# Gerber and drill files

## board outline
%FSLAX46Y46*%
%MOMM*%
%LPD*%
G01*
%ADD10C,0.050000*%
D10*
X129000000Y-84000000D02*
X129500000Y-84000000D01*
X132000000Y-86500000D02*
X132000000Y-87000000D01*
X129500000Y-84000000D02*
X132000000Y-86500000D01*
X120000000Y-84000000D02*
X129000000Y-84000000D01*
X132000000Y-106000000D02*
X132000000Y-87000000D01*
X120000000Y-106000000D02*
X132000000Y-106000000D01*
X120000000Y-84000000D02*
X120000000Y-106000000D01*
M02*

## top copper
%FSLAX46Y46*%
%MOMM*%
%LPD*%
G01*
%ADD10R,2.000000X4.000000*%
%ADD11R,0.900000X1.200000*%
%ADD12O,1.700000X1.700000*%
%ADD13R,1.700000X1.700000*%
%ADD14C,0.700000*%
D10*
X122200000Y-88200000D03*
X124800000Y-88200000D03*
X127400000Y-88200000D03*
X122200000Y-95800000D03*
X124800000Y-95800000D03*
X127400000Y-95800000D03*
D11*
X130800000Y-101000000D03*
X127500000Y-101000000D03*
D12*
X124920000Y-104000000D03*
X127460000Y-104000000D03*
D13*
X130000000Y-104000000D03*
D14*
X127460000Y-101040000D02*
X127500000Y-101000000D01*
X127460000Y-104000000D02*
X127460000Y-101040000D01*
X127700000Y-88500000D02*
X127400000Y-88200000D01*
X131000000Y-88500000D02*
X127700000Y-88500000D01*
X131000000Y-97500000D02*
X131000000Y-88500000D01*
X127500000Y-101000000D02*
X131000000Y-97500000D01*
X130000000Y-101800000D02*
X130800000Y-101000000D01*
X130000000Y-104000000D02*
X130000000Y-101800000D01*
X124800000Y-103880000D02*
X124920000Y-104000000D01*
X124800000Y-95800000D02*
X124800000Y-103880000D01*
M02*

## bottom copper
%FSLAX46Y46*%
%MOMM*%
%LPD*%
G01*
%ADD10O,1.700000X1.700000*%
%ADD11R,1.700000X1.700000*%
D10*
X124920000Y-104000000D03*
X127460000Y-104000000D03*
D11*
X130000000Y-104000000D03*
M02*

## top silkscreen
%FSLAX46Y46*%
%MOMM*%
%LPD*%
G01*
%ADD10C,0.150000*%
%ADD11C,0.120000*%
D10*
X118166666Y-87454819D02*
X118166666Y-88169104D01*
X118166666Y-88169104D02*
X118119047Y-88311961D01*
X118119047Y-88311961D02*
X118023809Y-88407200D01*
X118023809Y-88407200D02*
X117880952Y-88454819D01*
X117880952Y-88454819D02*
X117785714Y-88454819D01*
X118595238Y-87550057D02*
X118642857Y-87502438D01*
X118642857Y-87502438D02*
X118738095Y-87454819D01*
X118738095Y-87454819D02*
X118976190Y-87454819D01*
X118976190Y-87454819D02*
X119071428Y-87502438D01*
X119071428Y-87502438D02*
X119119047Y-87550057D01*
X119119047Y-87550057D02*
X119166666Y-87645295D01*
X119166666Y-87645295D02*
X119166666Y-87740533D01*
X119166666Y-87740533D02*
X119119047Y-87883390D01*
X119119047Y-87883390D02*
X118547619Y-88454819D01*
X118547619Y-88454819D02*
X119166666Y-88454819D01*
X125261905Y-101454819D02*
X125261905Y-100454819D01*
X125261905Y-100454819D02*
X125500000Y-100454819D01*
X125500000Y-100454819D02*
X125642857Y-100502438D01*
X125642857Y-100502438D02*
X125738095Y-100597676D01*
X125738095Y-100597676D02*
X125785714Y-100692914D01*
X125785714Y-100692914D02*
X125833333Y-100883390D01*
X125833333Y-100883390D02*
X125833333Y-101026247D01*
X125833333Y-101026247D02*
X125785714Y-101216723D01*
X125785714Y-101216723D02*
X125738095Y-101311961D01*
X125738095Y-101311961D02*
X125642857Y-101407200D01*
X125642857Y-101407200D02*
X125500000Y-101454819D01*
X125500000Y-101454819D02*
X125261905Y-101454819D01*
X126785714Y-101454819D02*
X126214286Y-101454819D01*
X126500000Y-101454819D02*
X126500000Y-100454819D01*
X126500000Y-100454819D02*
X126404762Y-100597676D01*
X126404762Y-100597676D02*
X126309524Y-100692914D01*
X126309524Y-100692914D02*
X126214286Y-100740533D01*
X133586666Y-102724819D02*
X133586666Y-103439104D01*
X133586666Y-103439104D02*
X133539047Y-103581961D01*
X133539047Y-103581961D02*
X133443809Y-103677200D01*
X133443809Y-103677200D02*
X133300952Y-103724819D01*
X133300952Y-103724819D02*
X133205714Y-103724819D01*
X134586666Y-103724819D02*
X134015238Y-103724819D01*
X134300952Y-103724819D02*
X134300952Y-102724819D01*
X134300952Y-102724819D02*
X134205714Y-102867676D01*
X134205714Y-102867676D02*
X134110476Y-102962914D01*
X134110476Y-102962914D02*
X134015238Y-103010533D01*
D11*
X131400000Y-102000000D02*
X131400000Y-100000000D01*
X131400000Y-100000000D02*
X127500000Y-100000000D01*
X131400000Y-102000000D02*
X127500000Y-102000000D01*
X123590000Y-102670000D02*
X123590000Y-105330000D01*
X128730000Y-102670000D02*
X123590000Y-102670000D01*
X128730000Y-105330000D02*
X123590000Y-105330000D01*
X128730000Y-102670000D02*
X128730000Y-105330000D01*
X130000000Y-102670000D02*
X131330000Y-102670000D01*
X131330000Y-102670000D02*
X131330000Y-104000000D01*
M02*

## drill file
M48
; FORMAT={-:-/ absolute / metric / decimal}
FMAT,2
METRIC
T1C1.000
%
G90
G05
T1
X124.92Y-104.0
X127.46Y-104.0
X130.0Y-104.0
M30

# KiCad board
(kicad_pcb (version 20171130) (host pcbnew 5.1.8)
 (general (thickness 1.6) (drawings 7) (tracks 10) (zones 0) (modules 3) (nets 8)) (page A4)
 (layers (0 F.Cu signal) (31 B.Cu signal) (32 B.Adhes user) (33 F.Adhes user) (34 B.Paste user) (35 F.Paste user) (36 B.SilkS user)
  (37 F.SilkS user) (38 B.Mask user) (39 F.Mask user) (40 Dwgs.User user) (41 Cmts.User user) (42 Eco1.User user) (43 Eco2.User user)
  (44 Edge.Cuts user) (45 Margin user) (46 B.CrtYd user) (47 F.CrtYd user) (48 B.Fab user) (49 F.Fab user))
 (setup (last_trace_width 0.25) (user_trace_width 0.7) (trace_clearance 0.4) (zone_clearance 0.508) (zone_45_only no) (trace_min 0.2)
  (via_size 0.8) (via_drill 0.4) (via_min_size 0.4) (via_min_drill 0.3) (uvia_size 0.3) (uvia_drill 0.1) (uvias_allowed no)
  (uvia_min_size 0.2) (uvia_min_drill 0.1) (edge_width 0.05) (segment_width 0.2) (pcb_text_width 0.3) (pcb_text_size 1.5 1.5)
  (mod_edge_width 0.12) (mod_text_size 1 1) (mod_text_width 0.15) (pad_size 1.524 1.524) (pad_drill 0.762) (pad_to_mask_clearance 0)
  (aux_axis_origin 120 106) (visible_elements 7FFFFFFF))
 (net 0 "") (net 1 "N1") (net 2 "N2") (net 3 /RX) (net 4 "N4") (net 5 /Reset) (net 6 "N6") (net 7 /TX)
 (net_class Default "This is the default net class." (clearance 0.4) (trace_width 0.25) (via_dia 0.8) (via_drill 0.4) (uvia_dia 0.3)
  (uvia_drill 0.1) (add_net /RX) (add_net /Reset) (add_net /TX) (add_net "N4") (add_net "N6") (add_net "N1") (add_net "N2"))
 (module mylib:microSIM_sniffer (layer F.Cu) (at 124 91)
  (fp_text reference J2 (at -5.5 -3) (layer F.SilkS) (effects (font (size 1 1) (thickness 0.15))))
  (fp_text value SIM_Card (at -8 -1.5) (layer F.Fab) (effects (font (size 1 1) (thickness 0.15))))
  (pad 5 smd rect (at -1.8 -2.8 270) (size 4 2) (layers F.Cu F.Paste F.Mask) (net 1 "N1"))
  (pad 6 smd rect (at 0.8 -2.8 270) (size 4 2) (layers F.Cu F.Paste F.Mask) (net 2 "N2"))
  (pad 7 smd rect (at 3.4 -2.8 270) (size 4 2) (layers F.Cu F.Paste F.Mask) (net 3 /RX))
  (pad 1 smd rect (at -1.8 4.8 270) (size 4 2) (layers F.Cu F.Paste F.Mask) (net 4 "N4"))
  (pad 2 smd rect (at 0.8 4.8 270) (size 4 2) (layers F.Cu F.Paste F.Mask) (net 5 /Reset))
  (pad 3 smd rect (at 3.4 4.8 270) (size 4 2) (layers F.Cu F.Paste F.Mask) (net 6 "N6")))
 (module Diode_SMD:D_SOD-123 (layer F.Cu) (at 129.15 101 180)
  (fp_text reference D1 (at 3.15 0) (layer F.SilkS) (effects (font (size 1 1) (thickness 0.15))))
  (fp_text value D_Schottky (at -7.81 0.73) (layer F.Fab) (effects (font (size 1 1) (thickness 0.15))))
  (fp_line (start -2.25 -1) (end -2.25 1) (layer F.SilkS) (width 0.12))
  (fp_line (start -2.25 1) (end 1.65 1) (layer F.SilkS) (width 0.12))
  (fp_line (start -2.25 -1) (end 1.65 -1) (layer F.SilkS) (width 0.12))
  (pad 1 smd rect (at -1.65 0 180) (size 0.9 1.2) (layers F.Cu F.Paste F.Mask) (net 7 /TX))
  (pad 2 smd rect (at 1.65 0 180) (size 0.9 1.2) (layers F.Cu F.Paste F.Mask) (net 3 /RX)))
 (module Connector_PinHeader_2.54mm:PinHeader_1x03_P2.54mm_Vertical (layer F.Cu) (at 130 104 270)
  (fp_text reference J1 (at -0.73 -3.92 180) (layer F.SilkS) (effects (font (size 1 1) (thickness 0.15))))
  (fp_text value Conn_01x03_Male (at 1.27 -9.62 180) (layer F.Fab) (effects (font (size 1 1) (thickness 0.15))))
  (fp_line (start -1.33 6.41) (end 1.33 6.41) (layer F.SilkS) (width 0.12))
  (fp_line (start -1.33 1.27) (end -1.33 6.41) (layer F.SilkS) (width 0.12))
  (fp_line (start 1.33 1.27) (end 1.33 6.41) (layer F.SilkS) (width 0.12))
  (fp_line (start -1.33 1.27) (end 1.33 1.27) (layer F.SilkS) (width 0.12))
  (fp_line (start -1.33 0) (end -1.33 -1.33) (layer F.SilkS) (width 0.12))
  (fp_line (start -1.33 -1.33) (end 0 -1.33) (layer F.SilkS) (width 0.12))
  (pad 3 thru_hole oval (at 0 5.08 270) (size 1.7 1.7) (drill 1) (layers *.Cu *.Mask) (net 5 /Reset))
  (pad 2 thru_hole oval (at 0 2.54 270) (size 1.7 1.7) (drill 1) (layers *.Cu *.Mask) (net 3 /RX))
  (pad 1 thru_hole rect (at 0 0 270) (size 1.7 1.7) (drill 1) (layers *.Cu *.Mask) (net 7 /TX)))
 (gr_line (start 129 84) (end 129.5 84) (layer Edge.Cuts) (width 0.05))
 (gr_line (start 132 86.5) (end 132 87) (layer Edge.Cuts) (width 0.05))
 (gr_line (start 129.5 84) (end 132 86.5) (layer Edge.Cuts) (width 0.05))
 (gr_line (start 120 84) (end 129 84) (layer Edge.Cuts) (width 0.05))
 (gr_line (start 132 106) (end 132 87) (layer Edge.Cuts) (width 0.05))
 (gr_line (start 120 106) (end 132 106) (layer Edge.Cuts) (width 0.05))
 (gr_line (start 120 84) (end 120 106) (layer Edge.Cuts) (width 0.05))
 (segment (start 127.46 101.04) (end 127.5 101) (width 0.7) (layer F.Cu) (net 3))
 (segment (start 127.46 104) (end 127.46 101.04) (width 0.7) (layer F.Cu) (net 3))
 (segment (start 127.7 88.5) (end 127.4 88.2) (width 0.7) (layer F.Cu) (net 3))
 (segment (start 131 88.5) (end 127.7 88.5) (width 0.7) (layer F.Cu) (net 3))
 (segment (start 131 97.5) (end 131 88.5) (width 0.7) (layer F.Cu) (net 3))
 (segment (start 127.5 101) (end 131 97.5) (width 0.7) (layer F.Cu) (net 3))
 (segment (start 130 101.8) (end 130.8 101) (width 0.7) (layer F.Cu) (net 7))
 (segment (start 130 104) (end 130 101.8) (width 0.7) (layer F.Cu) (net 7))
 (segment (start 124.8 103.88) (end 124.92 104) (width 0.7) (layer F.Cu) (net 5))
 (segment (start 124.8 95.8) (end 124.8 103.88) (width 0.7) (layer F.Cu) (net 5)))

